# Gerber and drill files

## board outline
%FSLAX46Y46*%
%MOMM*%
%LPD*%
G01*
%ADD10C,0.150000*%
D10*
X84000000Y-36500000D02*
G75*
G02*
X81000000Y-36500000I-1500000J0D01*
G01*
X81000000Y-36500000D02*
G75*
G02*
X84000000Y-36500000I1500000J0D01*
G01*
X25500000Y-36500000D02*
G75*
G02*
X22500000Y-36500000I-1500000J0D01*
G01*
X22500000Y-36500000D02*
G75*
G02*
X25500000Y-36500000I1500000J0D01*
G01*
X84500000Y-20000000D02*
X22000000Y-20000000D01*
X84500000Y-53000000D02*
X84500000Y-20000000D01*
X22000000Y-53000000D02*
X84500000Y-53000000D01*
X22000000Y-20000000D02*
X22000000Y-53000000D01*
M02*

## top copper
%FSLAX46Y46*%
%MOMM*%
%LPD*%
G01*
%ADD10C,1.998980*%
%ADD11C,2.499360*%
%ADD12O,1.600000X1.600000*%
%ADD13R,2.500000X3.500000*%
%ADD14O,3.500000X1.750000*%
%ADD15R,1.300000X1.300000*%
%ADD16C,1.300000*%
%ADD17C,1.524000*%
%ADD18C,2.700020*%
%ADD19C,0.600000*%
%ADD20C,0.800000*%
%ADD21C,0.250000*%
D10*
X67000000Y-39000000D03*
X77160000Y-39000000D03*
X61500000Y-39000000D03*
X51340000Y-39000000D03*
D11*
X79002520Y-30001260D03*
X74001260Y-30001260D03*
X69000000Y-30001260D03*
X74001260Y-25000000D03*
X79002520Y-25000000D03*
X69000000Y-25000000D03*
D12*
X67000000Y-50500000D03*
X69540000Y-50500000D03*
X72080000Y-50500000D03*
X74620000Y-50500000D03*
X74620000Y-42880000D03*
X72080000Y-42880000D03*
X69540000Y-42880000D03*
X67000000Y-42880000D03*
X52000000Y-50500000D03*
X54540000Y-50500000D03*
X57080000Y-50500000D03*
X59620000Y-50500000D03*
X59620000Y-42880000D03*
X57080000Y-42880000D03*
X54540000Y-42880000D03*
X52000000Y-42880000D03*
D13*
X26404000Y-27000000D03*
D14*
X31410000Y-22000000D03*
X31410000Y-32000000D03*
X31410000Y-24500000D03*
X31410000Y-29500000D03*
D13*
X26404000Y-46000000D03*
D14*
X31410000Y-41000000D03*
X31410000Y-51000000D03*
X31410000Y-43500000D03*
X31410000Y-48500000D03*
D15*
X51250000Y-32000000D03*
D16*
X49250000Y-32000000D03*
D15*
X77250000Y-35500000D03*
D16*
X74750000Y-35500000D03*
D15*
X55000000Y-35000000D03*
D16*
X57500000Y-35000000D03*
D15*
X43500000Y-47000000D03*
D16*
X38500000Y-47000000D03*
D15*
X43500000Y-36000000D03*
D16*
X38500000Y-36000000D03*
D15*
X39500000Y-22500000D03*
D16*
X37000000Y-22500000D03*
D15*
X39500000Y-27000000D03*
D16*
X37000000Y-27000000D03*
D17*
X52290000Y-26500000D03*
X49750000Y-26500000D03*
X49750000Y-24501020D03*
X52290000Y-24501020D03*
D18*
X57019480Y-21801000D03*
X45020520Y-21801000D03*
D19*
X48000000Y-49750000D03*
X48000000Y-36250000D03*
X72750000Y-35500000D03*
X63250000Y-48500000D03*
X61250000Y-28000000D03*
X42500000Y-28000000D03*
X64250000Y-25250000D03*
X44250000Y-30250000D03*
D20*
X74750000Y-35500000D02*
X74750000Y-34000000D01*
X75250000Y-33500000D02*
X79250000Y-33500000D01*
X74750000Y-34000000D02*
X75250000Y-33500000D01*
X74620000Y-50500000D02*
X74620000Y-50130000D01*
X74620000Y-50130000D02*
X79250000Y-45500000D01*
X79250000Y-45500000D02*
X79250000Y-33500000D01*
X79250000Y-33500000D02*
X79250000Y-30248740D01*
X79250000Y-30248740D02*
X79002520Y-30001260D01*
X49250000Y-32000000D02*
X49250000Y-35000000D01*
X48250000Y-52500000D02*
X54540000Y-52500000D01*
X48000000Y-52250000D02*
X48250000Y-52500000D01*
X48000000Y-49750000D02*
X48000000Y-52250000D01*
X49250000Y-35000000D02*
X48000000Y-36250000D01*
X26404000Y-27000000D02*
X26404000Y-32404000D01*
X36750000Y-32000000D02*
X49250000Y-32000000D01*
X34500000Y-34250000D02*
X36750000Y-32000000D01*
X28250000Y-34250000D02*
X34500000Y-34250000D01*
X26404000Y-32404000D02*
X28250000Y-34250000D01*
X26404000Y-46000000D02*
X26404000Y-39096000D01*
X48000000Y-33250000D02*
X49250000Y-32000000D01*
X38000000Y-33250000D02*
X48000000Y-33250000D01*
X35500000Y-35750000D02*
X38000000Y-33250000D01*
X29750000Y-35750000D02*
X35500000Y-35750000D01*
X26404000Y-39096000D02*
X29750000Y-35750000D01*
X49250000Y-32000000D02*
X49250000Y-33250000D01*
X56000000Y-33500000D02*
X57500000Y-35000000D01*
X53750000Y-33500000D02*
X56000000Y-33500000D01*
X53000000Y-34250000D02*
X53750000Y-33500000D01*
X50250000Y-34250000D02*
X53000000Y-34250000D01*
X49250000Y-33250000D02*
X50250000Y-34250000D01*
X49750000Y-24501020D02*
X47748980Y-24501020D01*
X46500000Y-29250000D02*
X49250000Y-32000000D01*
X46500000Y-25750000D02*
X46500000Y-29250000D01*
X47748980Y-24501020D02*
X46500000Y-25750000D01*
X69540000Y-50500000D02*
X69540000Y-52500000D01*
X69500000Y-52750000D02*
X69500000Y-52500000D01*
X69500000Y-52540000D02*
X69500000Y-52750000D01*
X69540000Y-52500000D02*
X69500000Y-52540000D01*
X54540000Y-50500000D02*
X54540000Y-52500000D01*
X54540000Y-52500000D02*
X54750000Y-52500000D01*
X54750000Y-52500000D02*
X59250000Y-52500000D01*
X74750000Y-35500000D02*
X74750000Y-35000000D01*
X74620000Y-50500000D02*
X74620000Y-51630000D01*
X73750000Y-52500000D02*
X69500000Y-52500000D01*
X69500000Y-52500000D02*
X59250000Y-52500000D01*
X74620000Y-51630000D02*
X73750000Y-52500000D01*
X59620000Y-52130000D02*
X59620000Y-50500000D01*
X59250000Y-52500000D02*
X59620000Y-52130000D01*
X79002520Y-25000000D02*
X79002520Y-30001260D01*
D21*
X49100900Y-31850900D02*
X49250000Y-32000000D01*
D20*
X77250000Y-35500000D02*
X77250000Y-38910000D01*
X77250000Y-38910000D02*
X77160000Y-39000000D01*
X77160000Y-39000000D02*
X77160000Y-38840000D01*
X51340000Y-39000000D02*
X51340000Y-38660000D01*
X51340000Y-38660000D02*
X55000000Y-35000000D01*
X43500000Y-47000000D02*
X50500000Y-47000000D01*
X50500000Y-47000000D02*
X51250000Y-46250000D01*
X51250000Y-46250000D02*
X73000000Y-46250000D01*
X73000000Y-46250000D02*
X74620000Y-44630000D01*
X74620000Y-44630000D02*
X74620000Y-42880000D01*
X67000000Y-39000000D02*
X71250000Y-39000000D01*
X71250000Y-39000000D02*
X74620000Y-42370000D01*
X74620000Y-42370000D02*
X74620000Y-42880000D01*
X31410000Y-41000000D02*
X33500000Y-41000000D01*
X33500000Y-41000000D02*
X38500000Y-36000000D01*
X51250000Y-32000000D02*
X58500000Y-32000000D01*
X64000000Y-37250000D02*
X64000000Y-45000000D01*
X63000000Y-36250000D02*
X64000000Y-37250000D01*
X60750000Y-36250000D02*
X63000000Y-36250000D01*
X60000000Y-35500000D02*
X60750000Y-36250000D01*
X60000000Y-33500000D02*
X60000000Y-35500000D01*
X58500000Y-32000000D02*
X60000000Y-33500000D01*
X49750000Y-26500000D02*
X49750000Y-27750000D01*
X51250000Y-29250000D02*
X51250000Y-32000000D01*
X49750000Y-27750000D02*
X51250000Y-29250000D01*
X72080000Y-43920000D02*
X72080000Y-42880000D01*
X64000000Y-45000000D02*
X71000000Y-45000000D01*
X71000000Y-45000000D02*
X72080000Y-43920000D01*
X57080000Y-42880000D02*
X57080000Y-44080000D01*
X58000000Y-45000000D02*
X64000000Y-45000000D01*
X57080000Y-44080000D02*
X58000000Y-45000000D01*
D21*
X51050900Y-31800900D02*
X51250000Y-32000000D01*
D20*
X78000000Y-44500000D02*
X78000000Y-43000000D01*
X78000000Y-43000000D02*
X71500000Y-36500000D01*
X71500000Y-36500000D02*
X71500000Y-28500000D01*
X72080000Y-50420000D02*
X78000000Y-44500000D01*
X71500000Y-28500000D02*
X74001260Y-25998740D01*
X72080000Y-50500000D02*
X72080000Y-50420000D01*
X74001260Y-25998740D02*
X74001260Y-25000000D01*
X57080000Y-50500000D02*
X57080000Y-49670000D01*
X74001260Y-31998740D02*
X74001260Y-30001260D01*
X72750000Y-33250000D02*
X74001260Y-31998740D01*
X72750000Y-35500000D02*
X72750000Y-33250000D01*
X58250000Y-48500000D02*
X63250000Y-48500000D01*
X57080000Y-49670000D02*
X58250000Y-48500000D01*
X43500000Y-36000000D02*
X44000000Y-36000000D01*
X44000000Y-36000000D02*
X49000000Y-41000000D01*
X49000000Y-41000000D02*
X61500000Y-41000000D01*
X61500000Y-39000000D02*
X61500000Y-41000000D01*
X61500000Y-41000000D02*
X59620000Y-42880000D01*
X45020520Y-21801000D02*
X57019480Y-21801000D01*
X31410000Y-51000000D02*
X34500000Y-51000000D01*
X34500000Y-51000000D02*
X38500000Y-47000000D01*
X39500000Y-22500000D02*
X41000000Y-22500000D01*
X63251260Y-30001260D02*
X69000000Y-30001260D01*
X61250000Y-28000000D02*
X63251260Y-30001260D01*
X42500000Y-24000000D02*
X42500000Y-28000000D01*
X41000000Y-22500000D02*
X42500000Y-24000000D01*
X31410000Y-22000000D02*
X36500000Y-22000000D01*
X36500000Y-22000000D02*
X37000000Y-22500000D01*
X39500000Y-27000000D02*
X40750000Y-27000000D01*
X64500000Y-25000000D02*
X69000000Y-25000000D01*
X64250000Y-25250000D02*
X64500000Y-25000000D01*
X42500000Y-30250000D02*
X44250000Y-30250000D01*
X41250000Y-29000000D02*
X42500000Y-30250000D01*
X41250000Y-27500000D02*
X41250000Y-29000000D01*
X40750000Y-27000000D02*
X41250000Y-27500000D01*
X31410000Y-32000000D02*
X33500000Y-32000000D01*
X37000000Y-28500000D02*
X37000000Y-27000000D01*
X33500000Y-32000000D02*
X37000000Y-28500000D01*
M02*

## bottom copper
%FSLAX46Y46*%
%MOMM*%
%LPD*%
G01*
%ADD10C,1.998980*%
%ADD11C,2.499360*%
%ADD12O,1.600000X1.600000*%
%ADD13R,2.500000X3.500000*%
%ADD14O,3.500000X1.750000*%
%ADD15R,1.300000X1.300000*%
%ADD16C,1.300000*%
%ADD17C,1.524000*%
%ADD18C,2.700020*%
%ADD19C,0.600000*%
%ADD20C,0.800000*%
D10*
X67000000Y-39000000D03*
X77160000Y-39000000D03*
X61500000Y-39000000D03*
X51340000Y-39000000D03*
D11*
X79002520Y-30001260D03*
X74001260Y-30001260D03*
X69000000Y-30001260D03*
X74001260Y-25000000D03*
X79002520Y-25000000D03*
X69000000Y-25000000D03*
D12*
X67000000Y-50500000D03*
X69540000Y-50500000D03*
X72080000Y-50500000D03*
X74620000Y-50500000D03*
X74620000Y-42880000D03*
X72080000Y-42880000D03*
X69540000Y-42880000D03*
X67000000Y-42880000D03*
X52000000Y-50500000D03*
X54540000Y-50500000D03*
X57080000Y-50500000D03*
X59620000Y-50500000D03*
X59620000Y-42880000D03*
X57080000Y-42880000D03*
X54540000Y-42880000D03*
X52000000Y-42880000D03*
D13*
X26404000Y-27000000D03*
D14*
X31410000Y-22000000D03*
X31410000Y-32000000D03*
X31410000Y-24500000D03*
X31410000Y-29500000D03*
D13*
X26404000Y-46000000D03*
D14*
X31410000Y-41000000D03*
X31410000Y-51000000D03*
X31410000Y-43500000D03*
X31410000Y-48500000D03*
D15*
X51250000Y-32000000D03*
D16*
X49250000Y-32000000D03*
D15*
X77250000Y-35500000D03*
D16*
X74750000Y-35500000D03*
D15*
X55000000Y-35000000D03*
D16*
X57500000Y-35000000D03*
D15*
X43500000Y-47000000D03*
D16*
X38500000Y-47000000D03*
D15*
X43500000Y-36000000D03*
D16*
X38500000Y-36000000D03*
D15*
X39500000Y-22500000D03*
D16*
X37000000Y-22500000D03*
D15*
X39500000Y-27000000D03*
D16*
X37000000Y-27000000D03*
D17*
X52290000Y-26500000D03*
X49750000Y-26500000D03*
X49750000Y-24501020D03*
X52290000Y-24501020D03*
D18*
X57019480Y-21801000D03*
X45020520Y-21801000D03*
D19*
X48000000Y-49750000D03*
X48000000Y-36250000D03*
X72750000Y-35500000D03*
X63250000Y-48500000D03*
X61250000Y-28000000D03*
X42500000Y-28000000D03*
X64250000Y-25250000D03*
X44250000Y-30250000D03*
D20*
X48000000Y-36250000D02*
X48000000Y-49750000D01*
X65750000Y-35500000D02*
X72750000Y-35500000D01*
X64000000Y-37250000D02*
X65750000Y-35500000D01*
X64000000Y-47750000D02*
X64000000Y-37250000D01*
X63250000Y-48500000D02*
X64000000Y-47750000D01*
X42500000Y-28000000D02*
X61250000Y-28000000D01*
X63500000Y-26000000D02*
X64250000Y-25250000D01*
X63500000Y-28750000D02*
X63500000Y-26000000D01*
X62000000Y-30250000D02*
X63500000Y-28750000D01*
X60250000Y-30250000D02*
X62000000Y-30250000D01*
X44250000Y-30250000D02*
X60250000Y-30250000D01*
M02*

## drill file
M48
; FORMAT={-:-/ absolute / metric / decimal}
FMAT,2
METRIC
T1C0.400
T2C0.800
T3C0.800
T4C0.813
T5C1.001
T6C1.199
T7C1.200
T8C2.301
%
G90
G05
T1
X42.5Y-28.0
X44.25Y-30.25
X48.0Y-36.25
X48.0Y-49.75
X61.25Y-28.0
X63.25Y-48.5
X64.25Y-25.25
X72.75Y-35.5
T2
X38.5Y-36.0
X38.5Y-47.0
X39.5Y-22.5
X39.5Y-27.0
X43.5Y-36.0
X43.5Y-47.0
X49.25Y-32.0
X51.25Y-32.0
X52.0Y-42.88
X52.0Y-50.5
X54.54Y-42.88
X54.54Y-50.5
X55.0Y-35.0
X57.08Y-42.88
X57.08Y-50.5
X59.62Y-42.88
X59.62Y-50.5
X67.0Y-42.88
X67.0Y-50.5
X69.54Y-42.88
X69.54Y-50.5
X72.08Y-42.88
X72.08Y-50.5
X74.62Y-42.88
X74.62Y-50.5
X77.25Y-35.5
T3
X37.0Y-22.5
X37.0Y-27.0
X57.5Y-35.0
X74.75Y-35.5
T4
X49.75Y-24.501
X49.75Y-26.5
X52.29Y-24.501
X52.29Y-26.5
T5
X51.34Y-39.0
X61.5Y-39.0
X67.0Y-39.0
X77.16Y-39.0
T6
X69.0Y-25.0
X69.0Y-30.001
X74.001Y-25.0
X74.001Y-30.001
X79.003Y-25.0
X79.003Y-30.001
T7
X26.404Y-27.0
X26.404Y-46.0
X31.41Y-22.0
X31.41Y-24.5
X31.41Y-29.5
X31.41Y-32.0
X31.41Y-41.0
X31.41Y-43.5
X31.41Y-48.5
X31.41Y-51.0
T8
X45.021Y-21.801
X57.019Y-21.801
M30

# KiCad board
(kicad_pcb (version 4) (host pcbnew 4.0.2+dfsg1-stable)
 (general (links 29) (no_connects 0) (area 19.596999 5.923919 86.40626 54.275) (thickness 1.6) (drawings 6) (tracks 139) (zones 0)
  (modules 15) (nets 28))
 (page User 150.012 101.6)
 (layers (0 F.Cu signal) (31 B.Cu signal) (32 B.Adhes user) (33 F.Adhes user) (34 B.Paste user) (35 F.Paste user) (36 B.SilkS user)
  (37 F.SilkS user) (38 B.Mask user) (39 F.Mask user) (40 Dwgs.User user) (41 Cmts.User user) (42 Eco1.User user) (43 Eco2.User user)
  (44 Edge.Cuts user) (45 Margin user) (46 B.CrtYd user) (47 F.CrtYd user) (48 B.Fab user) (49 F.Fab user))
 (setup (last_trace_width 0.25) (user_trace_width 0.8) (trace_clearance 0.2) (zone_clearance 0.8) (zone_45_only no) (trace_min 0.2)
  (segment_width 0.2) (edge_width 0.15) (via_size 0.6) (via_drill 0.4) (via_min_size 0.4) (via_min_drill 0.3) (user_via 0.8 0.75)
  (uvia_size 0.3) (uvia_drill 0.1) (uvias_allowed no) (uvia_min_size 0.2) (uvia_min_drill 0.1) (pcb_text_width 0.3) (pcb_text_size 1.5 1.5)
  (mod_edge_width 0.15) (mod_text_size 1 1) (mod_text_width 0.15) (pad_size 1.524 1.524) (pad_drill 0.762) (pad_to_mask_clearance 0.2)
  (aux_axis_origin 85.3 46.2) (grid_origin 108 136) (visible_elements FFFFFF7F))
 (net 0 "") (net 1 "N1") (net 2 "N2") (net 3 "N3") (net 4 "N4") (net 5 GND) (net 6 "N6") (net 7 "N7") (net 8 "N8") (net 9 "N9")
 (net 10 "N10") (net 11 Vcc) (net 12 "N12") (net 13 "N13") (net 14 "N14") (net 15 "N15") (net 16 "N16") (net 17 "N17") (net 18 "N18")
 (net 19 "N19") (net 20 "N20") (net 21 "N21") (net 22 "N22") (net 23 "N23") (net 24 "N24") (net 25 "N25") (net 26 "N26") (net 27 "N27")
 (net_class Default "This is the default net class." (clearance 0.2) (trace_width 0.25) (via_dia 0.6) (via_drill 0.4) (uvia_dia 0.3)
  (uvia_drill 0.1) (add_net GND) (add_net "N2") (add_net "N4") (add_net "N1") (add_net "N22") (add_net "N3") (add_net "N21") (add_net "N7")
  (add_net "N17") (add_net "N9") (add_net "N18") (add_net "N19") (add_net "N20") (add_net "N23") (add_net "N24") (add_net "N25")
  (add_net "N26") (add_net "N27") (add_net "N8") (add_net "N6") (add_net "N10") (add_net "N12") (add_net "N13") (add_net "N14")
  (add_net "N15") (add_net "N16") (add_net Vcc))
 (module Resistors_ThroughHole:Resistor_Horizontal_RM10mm (layer F.Cu) (at 67 39)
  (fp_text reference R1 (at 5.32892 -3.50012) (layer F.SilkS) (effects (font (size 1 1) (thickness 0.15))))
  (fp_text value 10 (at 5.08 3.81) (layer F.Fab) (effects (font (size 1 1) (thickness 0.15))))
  (pad 1 thru_hole circle (at 0 0) (size 1.99898 1.99898) (drill 1.00076) (layers *.Cu *.SilkS *.Mask) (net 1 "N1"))
  (pad 2 thru_hole circle (at 10.16 0) (size 1.99898 1.99898) (drill 1.00076) (layers *.Cu *.SilkS *.Mask) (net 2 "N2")))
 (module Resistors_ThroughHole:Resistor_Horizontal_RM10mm (layer F.Cu) (at 61.5 39 180)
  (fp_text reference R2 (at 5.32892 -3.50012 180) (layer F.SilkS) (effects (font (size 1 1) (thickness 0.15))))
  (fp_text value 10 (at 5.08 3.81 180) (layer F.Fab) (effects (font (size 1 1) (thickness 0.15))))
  (pad 1 thru_hole circle (at 0 0 180) (size 1.99898 1.99898) (drill 1.00076) (layers *.Cu *.SilkS *.Mask) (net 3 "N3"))
  (pad 2 thru_hole circle (at 10.16 0 180) (size 1.99898 1.99898) (drill 1.00076) (layers *.Cu *.SilkS *.Mask) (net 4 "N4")))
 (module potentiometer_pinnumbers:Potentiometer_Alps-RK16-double (layer F.Cu) (at 69 25 90)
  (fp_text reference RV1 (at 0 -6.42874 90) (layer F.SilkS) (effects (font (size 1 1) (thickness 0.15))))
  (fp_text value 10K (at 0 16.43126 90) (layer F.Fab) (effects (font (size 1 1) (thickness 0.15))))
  (pad 6 thru_hole circle (at -5.00126 10.00252 90) (size 2.49936 2.49936) (drill 1.19888) (layers *.Cu *.Mask F.SilkS) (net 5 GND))
  (pad 5 thru_hole circle (at -5.00126 5.00126 90) (size 2.49936 2.49936) (drill 1.19888) (layers *.Cu *.Mask F.SilkS) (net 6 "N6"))
  (pad 4 thru_hole circle (at -5.00126 0 90) (size 2.49936 2.49936) (drill 1.19888) (layers *.Cu *.Mask F.SilkS) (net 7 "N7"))
  (pad 2 thru_hole circle (at 0 5.00126 90) (size 2.49936 2.49936) (drill 1.19888) (layers *.Cu *.Mask F.SilkS) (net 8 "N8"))
  (pad 3 thru_hole circle (at 0 10.00252 90) (size 2.49936 2.49936) (drill 1.19888) (layers *.Cu *.Mask F.SilkS) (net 5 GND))
  (pad 1 thru_hole circle (at 0 0 90) (size 2.49936 2.49936) (drill 1.19888) (layers *.Cu *.Mask F.SilkS) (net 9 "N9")))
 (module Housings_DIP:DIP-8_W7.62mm (layer F.Cu) (at 67 50.5 90)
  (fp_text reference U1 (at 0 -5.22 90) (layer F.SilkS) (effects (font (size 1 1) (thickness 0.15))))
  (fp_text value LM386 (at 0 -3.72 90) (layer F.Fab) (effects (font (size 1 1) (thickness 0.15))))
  (pad 1 thru_hole oval (at 0 0 90) (size 1.6 1.6) (drill 0.8) (layers *.Cu *.Mask F.SilkS) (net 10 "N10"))
  (pad 2 thru_hole oval (at 0 2.54 90) (size 1.6 1.6) (drill 0.8) (layers *.Cu *.Mask F.SilkS) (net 5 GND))
  (pad 3 thru_hole oval (at 0 5.08 90) (size 1.6 1.6) (drill 0.8) (layers *.Cu *.Mask F.SilkS) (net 8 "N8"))
  (pad 4 thru_hole oval (at 0 7.62 90) (size 1.6 1.6) (drill 0.8) (layers *.Cu *.Mask F.SilkS) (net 5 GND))
  (pad 5 thru_hole oval (at 7.62 7.62 90) (size 1.6 1.6) (drill 0.8) (layers *.Cu *.Mask F.SilkS) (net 1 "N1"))
  (pad 6 thru_hole oval (at 7.62 5.08 90) (size 1.6 1.6) (drill 0.8) (layers *.Cu *.Mask F.SilkS) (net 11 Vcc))
  (pad 7 thru_hole oval (at 7.62 2.54 90) (size 1.6 1.6) (drill 0.8) (layers *.Cu *.Mask F.SilkS) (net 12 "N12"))
  (pad 8 thru_hole oval (at 7.62 0 90) (size 1.6 1.6) (drill 0.8) (layers *.Cu *.Mask F.SilkS) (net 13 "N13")))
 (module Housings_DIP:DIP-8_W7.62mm (layer F.Cu) (at 52 50.5 90)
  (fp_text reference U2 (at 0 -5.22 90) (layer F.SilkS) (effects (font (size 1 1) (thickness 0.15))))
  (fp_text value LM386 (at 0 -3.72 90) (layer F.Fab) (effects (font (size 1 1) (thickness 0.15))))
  (pad 1 thru_hole oval (at 0 0 90) (size 1.6 1.6) (drill 0.8) (layers *.Cu *.Mask F.SilkS) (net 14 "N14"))
  (pad 2 thru_hole oval (at 0 2.54 90) (size 1.6 1.6) (drill 0.8) (layers *.Cu *.Mask F.SilkS) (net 5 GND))
  (pad 3 thru_hole oval (at 0 5.08 90) (size 1.6 1.6) (drill 0.8) (layers *.Cu *.Mask F.SilkS) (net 6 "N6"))
  (pad 4 thru_hole oval (at 0 7.62 90) (size 1.6 1.6) (drill 0.8) (layers *.Cu *.Mask F.SilkS) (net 5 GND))
  (pad 5 thru_hole oval (at 7.62 7.62 90) (size 1.6 1.6) (drill 0.8) (layers *.Cu *.Mask F.SilkS) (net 3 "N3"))
  (pad 6 thru_hole oval (at 7.62 5.08 90) (size 1.6 1.6) (drill 0.8) (layers *.Cu *.Mask F.SilkS) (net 11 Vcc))
  (pad 7 thru_hole oval (at 7.62 2.54 90) (size 1.6 1.6) (drill 0.8) (layers *.Cu *.Mask F.SilkS) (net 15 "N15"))
  (pad 8 thru_hole oval (at 7.62 0 90) (size 1.6 1.6) (drill 0.8) (layers *.Cu *.Mask F.SilkS) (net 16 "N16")))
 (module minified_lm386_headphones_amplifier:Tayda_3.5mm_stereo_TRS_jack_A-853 (layer F.Cu) (at 28 27 90)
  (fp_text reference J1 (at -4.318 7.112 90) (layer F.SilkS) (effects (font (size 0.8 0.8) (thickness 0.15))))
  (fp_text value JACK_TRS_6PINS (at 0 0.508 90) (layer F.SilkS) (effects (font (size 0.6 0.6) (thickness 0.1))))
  (pad 1 thru_hole rect (at 0 -1.596 90) (size 3.5 2.5) (drill 1.2) (layers *.Cu *.Mask F.SilkS) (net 5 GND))
  (pad 2 thru_hole oval (at 5 3.41 90) (size 1.75 3.5) (drill 1.2) (layers *.Cu *.Mask F.SilkS) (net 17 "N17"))
  (pad 3 thru_hole oval (at -5 3.41 90) (size 1.75 3.5) (drill 1.2) (layers *.Cu *.Mask F.SilkS) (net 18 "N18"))
  (pad 4 thru_hole oval (at 2.5 3.41 90) (size 1.75 3.5) (drill 1.2) (layers *.Cu *.Mask F.SilkS) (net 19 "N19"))
  (pad 5 thru_hole oval (at -2.5 3.41 90) (size 1.75 3.5) (drill 1.2) (layers *.Cu *.Mask F.SilkS) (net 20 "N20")))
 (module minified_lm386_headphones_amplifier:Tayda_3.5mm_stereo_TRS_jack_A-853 (layer F.Cu) (at 28 46 90)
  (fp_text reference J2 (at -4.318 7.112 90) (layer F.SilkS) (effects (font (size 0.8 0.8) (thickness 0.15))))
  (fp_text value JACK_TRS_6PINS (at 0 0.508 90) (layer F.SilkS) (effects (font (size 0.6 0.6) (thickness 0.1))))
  (pad 1 thru_hole rect (at 0 -1.596 90) (size 3.5 2.5) (drill 1.2) (layers *.Cu *.Mask F.SilkS) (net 5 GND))
  (pad 2 thru_hole oval (at 5 3.41 90) (size 1.75 3.5) (drill 1.2) (layers *.Cu *.Mask F.SilkS) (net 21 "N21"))
  (pad 3 thru_hole oval (at -5 3.41 90) (size 1.75 3.5) (drill 1.2) (layers *.Cu *.Mask F.SilkS) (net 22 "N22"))
  (pad 4 thru_hole oval (at 2.5 3.41 90) (size 1.75 3.5) (drill 1.2) (layers *.Cu *.Mask F.SilkS) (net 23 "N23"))
  (pad 5 thru_hole oval (at -2.5 3.41 90) (size 1.75 3.5) (drill 1.2) (layers *.Cu *.Mask F.SilkS) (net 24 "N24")))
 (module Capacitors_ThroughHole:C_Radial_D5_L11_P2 (layer F.Cu) (at 51.25 32 180)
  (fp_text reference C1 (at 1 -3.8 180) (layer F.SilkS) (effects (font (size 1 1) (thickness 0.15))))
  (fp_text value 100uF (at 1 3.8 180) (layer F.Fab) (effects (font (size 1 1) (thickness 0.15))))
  (pad 1 thru_hole rect (at 0 0 180) (size 1.3 1.3) (drill 0.8) (layers *.Cu *.Mask F.SilkS) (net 11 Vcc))
  (pad 2 thru_hole circle (at 2 0 180) (size 1.3 1.3) (drill 0.8) (layers *.Cu *.Mask F.SilkS) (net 5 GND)))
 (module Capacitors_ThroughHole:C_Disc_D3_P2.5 (layer F.Cu) (at 77.25 35.5 180)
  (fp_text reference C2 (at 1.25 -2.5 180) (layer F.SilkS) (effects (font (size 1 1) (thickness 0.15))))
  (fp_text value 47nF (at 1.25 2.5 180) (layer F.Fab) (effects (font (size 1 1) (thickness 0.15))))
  (pad 1 thru_hole rect (at 0 0 180) (size 1.3 1.3) (drill 0.8) (layers *.Cu *.Mask F.SilkS) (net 2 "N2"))
  (pad 2 thru_hole circle (at 2.5 0 180) (size 1.3 1.3) (drill 0.8001) (layers *.Cu *.Mask F.SilkS) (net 5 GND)))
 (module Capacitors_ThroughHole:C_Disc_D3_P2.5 (layer F.Cu) (at 55 35)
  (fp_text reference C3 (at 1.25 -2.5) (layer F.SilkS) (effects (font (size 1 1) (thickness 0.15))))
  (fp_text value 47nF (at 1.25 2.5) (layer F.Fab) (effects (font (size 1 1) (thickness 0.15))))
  (pad 1 thru_hole rect (at 0 0) (size 1.3 1.3) (drill 0.8) (layers *.Cu *.Mask F.SilkS) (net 4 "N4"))
  (pad 2 thru_hole circle (at 2.5 0) (size 1.3 1.3) (drill 0.8001) (layers *.Cu *.Mask F.SilkS) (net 5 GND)))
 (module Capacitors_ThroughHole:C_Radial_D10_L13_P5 (layer F.Cu) (at 43.5 47 180)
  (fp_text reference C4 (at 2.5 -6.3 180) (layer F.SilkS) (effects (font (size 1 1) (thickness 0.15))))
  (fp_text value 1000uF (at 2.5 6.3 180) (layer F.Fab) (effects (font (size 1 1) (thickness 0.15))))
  (pad 1 thru_hole rect (at 0 0 180) (size 1.3 1.3) (drill 0.8) (layers *.Cu *.Mask F.SilkS) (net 1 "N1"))
  (pad 2 thru_hole circle (at 5 0 180) (size 1.3 1.3) (drill 0.8) (layers *.Cu *.Mask F.SilkS) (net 22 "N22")))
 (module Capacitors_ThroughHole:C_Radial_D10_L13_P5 (layer F.Cu) (at 43.5 36 180)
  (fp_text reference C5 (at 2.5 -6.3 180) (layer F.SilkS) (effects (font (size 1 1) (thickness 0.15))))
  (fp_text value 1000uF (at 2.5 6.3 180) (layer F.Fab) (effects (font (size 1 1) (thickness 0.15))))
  (pad 1 thru_hole rect (at 0 0 180) (size 1.3 1.3) (drill 0.8) (layers *.Cu *.Mask F.SilkS) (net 3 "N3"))
  (pad 2 thru_hole circle (at 5 0 180) (size 1.3 1.3) (drill 0.8) (layers *.Cu *.Mask F.SilkS) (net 21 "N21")))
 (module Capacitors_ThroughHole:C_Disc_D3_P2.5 (layer F.Cu) (at 39.5 22.5 180)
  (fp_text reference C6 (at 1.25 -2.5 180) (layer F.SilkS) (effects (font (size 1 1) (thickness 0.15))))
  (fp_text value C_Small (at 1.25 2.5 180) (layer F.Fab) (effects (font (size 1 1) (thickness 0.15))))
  (pad 1 thru_hole rect (at 0 0 180) (size 1.3 1.3) (drill 0.8) (layers *.Cu *.Mask F.SilkS) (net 7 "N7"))
  (pad 2 thru_hole circle (at 2.5 0 180) (size 1.3 1.3) (drill 0.8001) (layers *.Cu *.Mask F.SilkS) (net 17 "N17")))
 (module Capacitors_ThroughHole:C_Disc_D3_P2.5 (layer F.Cu) (at 39.5 27 180)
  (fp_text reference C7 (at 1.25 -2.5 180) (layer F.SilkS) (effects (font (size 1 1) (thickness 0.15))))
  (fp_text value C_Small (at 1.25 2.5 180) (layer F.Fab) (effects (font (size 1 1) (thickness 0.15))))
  (pad 1 thru_hole rect (at 0 0 180) (size 1.3 1.3) (drill 0.8) (layers *.Cu *.Mask F.SilkS) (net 9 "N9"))
  (pad 2 thru_hole circle (at 2.5 0 180) (size 1.3 1.3) (drill 0.8001) (layers *.Cu *.Mask F.SilkS) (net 18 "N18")))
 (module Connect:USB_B (layer F.Cu) (at 49.75 26.5 90)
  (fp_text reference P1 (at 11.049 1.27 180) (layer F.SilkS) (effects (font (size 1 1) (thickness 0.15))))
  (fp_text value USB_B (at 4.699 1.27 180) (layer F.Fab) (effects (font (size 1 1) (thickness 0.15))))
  (pad 2 thru_hole circle (at 0 2.54) (size 1.524 1.524) (drill 0.8128) (layers *.Cu *.Mask F.SilkS) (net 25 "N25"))
  (pad 1 thru_hole circle (at 0 0) (size 1.524 1.524) (drill 0.8128) (layers *.Cu *.Mask F.SilkS) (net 11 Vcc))
  (pad 4 thru_hole circle (at 1.99898 0) (size 1.524 1.524) (drill 0.8128) (layers *.Cu *.Mask F.SilkS) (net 5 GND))
  (pad 3 thru_hole circle (at 1.99898 2.54) (size 1.524 1.524) (drill 0.8128) (layers *.Cu *.Mask F.SilkS) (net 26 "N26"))
  (pad 5 thru_hole circle (at 4.699 7.26948) (size 2.70002 2.70002) (drill 2.30124) (layers *.Cu *.Mask F.SilkS) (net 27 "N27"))
  (pad 5 thru_hole circle (at 4.699 -4.72948) (size 2.70002 2.70002) (drill 2.30124) (layers *.Cu *.Mask F.SilkS) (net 27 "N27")))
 (gr_circle (center 82.5 36.5) (end 84 36.5) (layer Edge.Cuts) (width 0.15))
 (gr_circle (center 24 36.5) (end 22.5 36.5) (layer Edge.Cuts) (width 0.15))
 (gr_line (start 84.5 20) (end 22 20) (angle 90) (layer Edge.Cuts) (width 0.15))
 (gr_line (start 84.5 53) (end 84.5 20) (angle 90) (layer Edge.Cuts) (width 0.15))
 (gr_line (start 22 53) (end 84.5 53) (angle 90) (layer Edge.Cuts) (width 0.15))
 (gr_line (start 22 20) (end 22 53) (angle 90) (layer Edge.Cuts) (width 0.15))
 (segment (start 74.75 35.5) (end 74.75 34) (width 0.8) (layer F.Cu) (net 5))
 (segment (start 75.25 33.5) (end 79.25 33.5) (width 0.8) (layer F.Cu) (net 5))
 (segment (start 74.75 34) (end 75.25 33.5) (width 0.8) (layer F.Cu) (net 5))
 (segment (start 74.62 50.5) (end 74.62 50.13) (width 0.8) (layer F.Cu) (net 5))
 (segment (start 74.62 50.13) (end 79.25 45.5) (width 0.8) (layer F.Cu) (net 5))
 (segment (start 79.25 45.5) (end 79.25 33.5) (width 0.8) (layer F.Cu) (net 5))
 (segment (start 79.25 33.5) (end 79.25 30.24874) (width 0.8) (layer F.Cu) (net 5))
 (segment (start 79.25 30.24874) (end 79.00252 30.00126) (width 0.8) (layer F.Cu) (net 5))
 (segment (start 49.25 32) (end 49.25 35) (width 0.8) (layer F.Cu) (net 5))
 (segment (start 48.25 52.5) (end 54.54 52.5) (width 0.8) (layer F.Cu) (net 5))
 (segment (start 48 52.25) (end 48.25 52.5) (width 0.8) (layer F.Cu) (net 5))
 (segment (start 48 49.75) (end 48 52.25) (width 0.8) (layer F.Cu) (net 5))
 (via (at 48 49.75) (size 0.6) (drill 0.4) (layers F.Cu B.Cu) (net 5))
 (segment (start 48 36.25) (end 48 49.75) (width 0.8) (layer B.Cu) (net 5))
 (via (at 48 36.25) (size 0.6) (drill 0.4) (layers F.Cu B.Cu) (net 5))
 (segment (start 49.25 35) (end 48 36.25) (width 0.8) (layer F.Cu) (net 5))
 (segment (start 26.404 27) (end 26.404 32.404) (width 0.8) (layer F.Cu) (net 5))
 (segment (start 36.75 32) (end 49.25 32) (width 0.8) (layer F.Cu) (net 5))
 (segment (start 34.5 34.25) (end 36.75 32) (width 0.8) (layer F.Cu) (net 5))
 (segment (start 28.25 34.25) (end 34.5 34.25) (width 0.8) (layer F.Cu) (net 5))
 (segment (start 26.404 32.404) (end 28.25 34.25) (width 0.8) (layer F.Cu) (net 5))
 (segment (start 26.404 46) (end 26.404 39.096) (width 0.8) (layer F.Cu) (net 5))
 (segment (start 48 33.25) (end 49.25 32) (width 0.8) (layer F.Cu) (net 5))
 (segment (start 38 33.25) (end 48 33.25) (width 0.8) (layer F.Cu) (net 5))
 (segment (start 35.5 35.75) (end 38 33.25) (width 0.8) (layer F.Cu) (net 5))
 (segment (start 29.75 35.75) (end 35.5 35.75) (width 0.8) (layer F.Cu) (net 5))
 (segment (start 26.404 39.096) (end 29.75 35.75) (width 0.8) (layer F.Cu) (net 5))
 (segment (start 49.25 32) (end 49.25 33.25) (width 0.8) (layer F.Cu) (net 5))
 (segment (start 56 33.5) (end 57.5 35) (width 0.8) (layer F.Cu) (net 5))
 (segment (start 53.75 33.5) (end 56 33.5) (width 0.8) (layer F.Cu) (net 5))
 (segment (start 53 34.25) (end 53.75 33.5) (width 0.8) (layer F.Cu) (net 5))
 (segment (start 50.25 34.25) (end 53 34.25) (width 0.8) (layer F.Cu) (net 5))
 (segment (start 49.25 33.25) (end 50.25 34.25) (width 0.8) (layer F.Cu) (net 5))
 (segment (start 49.75 24.50102) (end 47.74898 24.50102) (width 0.8) (layer F.Cu) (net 5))
 (segment (start 46.5 29.25) (end 49.25 32) (width 0.8) (layer F.Cu) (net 5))
 (segment (start 46.5 25.75) (end 46.5 29.25) (width 0.8) (layer F.Cu) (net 5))
 (segment (start 47.74898 24.50102) (end 46.5 25.75) (width 0.8) (layer F.Cu) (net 5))
 (segment (start 69.54 50.5) (end 69.54 52.5) (width 0.8) (layer F.Cu) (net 5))
 (segment (start 69.5 52.75) (end 69.5 52.5) (width 0.8) (layer F.Cu) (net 5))
 (segment (start 69.5 52.54) (end 69.5 52.75) (width 0.8) (layer F.Cu) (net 5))
 (segment (start 69.54 52.5) (end 69.5 52.54) (width 0.8) (layer F.Cu) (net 5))
 (segment (start 54.54 50.5) (end 54.54 52.5) (width 0.8) (layer F.Cu) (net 5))
 (segment (start 54.54 52.5) (end 54.75 52.5) (width 0.8) (layer F.Cu) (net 5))
 (segment (start 54.75 52.5) (end 59.25 52.5) (width 0.8) (layer F.Cu) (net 5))
 (segment (start 74.75 35.5) (end 74.75 35) (width 0.8) (layer F.Cu) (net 5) (status 30))
 (segment (start 74.62 50.5) (end 74.62 51.63) (width 0.8) (layer F.Cu) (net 5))
 (segment (start 73.75 52.5) (end 69.5 52.5) (width 0.8) (layer F.Cu) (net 5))
 (segment (start 69.5 52.5) (end 59.25 52.5) (width 0.8) (layer F.Cu) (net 5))
 (segment (start 74.62 51.63) (end 73.75 52.5) (width 0.8) (layer F.Cu) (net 5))
 (segment (start 59.62 52.13) (end 59.62 50.5) (width 0.8) (layer F.Cu) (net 5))
 (segment (start 59.25 52.5) (end 59.62 52.13) (width 0.8) (layer F.Cu) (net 5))
 (segment (start 79.00252 25) (end 79.00252 30.00126) (width 0.8) (layer F.Cu) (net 5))
 (segment (start 49.1009 31.8509) (end 49.25 32) (width 0.25) (layer F.Cu) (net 5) (status 30))
 (segment (start 77.25 35.5) (end 77.25 38.91) (width 0.8) (layer F.Cu) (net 2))
 (segment (start 77.25 38.91) (end 77.16 39) (width 0.8) (layer F.Cu) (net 2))
 (segment (start 77.16 39) (end 77.16 38.84) (width 0.8) (layer F.Cu) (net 2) (status 30))
 (segment (start 51.34 39) (end 51.34 38.66) (width 0.8) (layer F.Cu) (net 4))
 (segment (start 51.34 38.66) (end 55 35) (width 0.8) (layer F.Cu) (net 4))
 (segment (start 43.5 47) (end 50.5 47) (width 0.8) (layer F.Cu) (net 1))
 (segment (start 50.5 47) (end 51.25 46.25) (width 0.8) (layer F.Cu) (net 1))
 (segment (start 51.25 46.25) (end 73 46.25) (width 0.8) (layer F.Cu) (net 1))
 (segment (start 73 46.25) (end 74.62 44.63) (width 0.8) (layer F.Cu) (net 1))
 (segment (start 74.62 44.63) (end 74.62 42.88) (width 0.8) (layer F.Cu) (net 1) (status 20))
 (segment (start 67 39) (end 71.25 39) (width 0.8) (layer F.Cu) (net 1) (status 10))
 (segment (start 71.25 39) (end 74.62 42.37) (width 0.8) (layer F.Cu) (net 1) (status 20))
 (segment (start 74.62 42.37) (end 74.62 42.88) (width 0.8) (layer F.Cu) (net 1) (status 30))
 (segment (start 31.41 41) (end 33.5 41) (width 0.8) (layer F.Cu) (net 21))
 (segment (start 33.5 41) (end 38.5 36) (width 0.8) (layer F.Cu) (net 21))
 (segment (start 51.25 32) (end 58.5 32) (width 0.8) (layer F.Cu) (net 11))
 (segment (start 64 37.25) (end 64 45) (width 0.8) (layer F.Cu) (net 11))
 (segment (start 63 36.25) (end 64 37.25) (width 0.8) (layer F.Cu) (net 11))
 (segment (start 60.75 36.25) (end 63 36.25) (width 0.8) (layer F.Cu) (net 11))
 (segment (start 60 35.5) (end 60.75 36.25) (width 0.8) (layer F.Cu) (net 11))
 (segment (start 60 33.5) (end 60 35.5) (width 0.8) (layer F.Cu) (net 11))
 (segment (start 58.5 32) (end 60 33.5) (width 0.8) (layer F.Cu) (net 11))
 (segment (start 49.75 26.5) (end 49.75 27.75) (width 0.8) (layer F.Cu) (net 11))
 (segment (start 51.25 29.25) (end 51.25 32) (width 0.8) (layer F.Cu) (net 11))
 (segment (start 49.75 27.75) (end 51.25 29.25) (width 0.8) (layer F.Cu) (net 11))
 (segment (start 72.08 43.92) (end 72.08 42.88) (width 0.8) (layer F.Cu) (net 11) (status 20))
 (segment (start 64 45) (end 71 45) (width 0.8) (layer F.Cu) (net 11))
 (segment (start 71 45) (end 72.08 43.92) (width 0.8) (layer F.Cu) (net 11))
 (segment (start 57.08 42.88) (end 57.08 44.08) (width 0.8) (layer F.Cu) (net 11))
 (segment (start 58 45) (end 64 45) (width 0.8) (layer F.Cu) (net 11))
 (segment (start 57.08 44.08) (end 58 45) (width 0.8) (layer F.Cu) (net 11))
 (segment (start 51.0509 31.8009) (end 51.25 32) (width 0.25) (layer F.Cu) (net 11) (status 30))
 (segment (start 78 44.5) (end 78 43) (width 0.8) (layer F.Cu) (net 8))
 (segment (start 78 43) (end 71.5 36.5) (width 0.8) (layer F.Cu) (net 8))
 (segment (start 71.5 36.5) (end 71.5 28.5) (width 0.8) (layer F.Cu) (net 8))
 (segment (start 72.08 50.42) (end 78 44.5) (width 0.8) (layer F.Cu) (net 8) (status 10))
 (segment (start 71.5 28.5) (end 74.00126 25.99874) (width 0.8) (layer F.Cu) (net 8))
 (segment (start 72.08 50.5) (end 72.08 50.42) (width 0.8) (layer F.Cu) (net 8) (status 30))
 (segment (start 74.00126 25.99874) (end 74.00126 25) (width 0.8) (layer F.Cu) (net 8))
 (segment (start 57.08 50.5) (end 57.08 49.67) (width 0.8) (layer F.Cu) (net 6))
 (segment (start 74.00126 31.99874) (end 74.00126 30.00126) (width 0.8) (layer F.Cu) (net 6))
 (segment (start 72.75 33.25) (end 74.00126 31.99874) (width 0.8) (layer F.Cu) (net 6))
 (segment (start 72.75 35.5) (end 72.75 33.25) (width 0.8) (layer F.Cu) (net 6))
 (via (at 72.75 35.5) (size 0.6) (drill 0.4) (layers F.Cu B.Cu) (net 6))
 (segment (start 65.75 35.5) (end 72.75 35.5) (width 0.8) (layer B.Cu) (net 6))
 (segment (start 64 37.25) (end 65.75 35.5) (width 0.8) (layer B.Cu) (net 6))
 (segment (start 64 47.75) (end 64 37.25) (width 0.8) (layer B.Cu) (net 6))
 (segment (start 63.25 48.5) (end 64 47.75) (width 0.8) (layer B.Cu) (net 6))
 (via (at 63.25 48.5) (size 0.6) (drill 0.4) (layers F.Cu B.Cu) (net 6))
 (segment (start 58.25 48.5) (end 63.25 48.5) (width 0.8) (layer F.Cu) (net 6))
 (segment (start 57.08 49.67) (end 58.25 48.5) (width 0.8) (layer F.Cu) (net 6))
 (segment (start 43.5 36) (end 44 36) (width 0.8) (layer F.Cu) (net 3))
 (segment (start 44 36) (end 49 41) (width 0.8) (layer F.Cu) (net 3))
 (segment (start 49 41) (end 61.5 41) (width 0.8) (layer F.Cu) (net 3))
 (segment (start 61.5 39) (end 61.5 41) (width 0.8) (layer F.Cu) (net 3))
 (segment (start 61.5 41) (end 59.62 42.88) (width 0.8) (layer F.Cu) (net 3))
 (segment (start 45.02052 21.801) (end 57.01948 21.801) (width 0.8) (layer F.Cu) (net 27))
 (segment (start 31.41 51) (end 34.5 51) (width 0.8) (layer F.Cu) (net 22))
 (segment (start 34.5 51) (end 38.5 47) (width 0.8) (layer F.Cu) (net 22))
 (segment (start 39.5 22.5) (end 41 22.5) (width 0.8) (layer F.Cu) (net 7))
 (segment (start 63.25126 30.00126) (end 69 30.00126) (width 0.8) (layer F.Cu) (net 7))
 (segment (start 61.25 28) (end 63.25126 30.00126) (width 0.8) (layer F.Cu) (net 7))
 (via (at 61.25 28) (size 0.6) (drill 0.4) (layers F.Cu B.Cu) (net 7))
 (segment (start 42.5 28) (end 61.25 28) (width 0.8) (layer B.Cu) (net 7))
 (via (at 42.5 28) (size 0.6) (drill 0.4) (layers F.Cu B.Cu) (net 7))
 (segment (start 42.5 24) (end 42.5 28) (width 0.8) (layer F.Cu) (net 7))
 (segment (start 41 22.5) (end 42.5 24) (width 0.8) (layer F.Cu) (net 7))
 (segment (start 31.41 22) (end 36.5 22) (width 0.8) (layer F.Cu) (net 17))
 (segment (start 36.5 22) (end 37 22.5) (width 0.8) (layer F.Cu) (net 17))
 (segment (start 39.5 27) (end 40.75 27) (width 0.8) (layer F.Cu) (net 9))
 (segment (start 64.5 25) (end 69 25) (width 0.8) (layer F.Cu) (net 9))
 (segment (start 64.25 25.25) (end 64.5 25) (width 0.8) (layer F.Cu) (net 9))
 (via (at 64.25 25.25) (size 0.6) (drill 0.4) (layers F.Cu B.Cu) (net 9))
 (segment (start 63.5 26) (end 64.25 25.25) (width 0.8) (layer B.Cu) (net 9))
 (segment (start 63.5 28.75) (end 63.5 26) (width 0.8) (layer B.Cu) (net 9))
 (segment (start 62 30.25) (end 63.5 28.75) (width 0.8) (layer B.Cu) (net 9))
 (segment (start 60.25 30.25) (end 62 30.25) (width 0.8) (layer B.Cu) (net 9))
 (segment (start 44.25 30.25) (end 60.25 30.25) (width 0.8) (layer B.Cu) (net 9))
 (via (at 44.25 30.25) (size 0.6) (drill 0.4) (layers F.Cu B.Cu) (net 9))
 (segment (start 42.5 30.25) (end 44.25 30.25) (width 0.8) (layer F.Cu) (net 9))
 (segment (start 41.25 29) (end 42.5 30.25) (width 0.8) (layer F.Cu) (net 9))
 (segment (start 41.25 27.5) (end 41.25 29) (width 0.8) (layer F.Cu) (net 9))
 (segment (start 40.75 27) (end 41.25 27.5) (width 0.8) (layer F.Cu) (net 9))
 (segment (start 31.41 32) (end 33.5 32) (width 0.8) (layer F.Cu) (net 18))
 (segment (start 37 28.5) (end 37 27) (width 0.8) (layer F.Cu) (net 18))
 (segment (start 33.5 32) (end 37 28.5) (width 0.8) (layer F.Cu) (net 18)))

